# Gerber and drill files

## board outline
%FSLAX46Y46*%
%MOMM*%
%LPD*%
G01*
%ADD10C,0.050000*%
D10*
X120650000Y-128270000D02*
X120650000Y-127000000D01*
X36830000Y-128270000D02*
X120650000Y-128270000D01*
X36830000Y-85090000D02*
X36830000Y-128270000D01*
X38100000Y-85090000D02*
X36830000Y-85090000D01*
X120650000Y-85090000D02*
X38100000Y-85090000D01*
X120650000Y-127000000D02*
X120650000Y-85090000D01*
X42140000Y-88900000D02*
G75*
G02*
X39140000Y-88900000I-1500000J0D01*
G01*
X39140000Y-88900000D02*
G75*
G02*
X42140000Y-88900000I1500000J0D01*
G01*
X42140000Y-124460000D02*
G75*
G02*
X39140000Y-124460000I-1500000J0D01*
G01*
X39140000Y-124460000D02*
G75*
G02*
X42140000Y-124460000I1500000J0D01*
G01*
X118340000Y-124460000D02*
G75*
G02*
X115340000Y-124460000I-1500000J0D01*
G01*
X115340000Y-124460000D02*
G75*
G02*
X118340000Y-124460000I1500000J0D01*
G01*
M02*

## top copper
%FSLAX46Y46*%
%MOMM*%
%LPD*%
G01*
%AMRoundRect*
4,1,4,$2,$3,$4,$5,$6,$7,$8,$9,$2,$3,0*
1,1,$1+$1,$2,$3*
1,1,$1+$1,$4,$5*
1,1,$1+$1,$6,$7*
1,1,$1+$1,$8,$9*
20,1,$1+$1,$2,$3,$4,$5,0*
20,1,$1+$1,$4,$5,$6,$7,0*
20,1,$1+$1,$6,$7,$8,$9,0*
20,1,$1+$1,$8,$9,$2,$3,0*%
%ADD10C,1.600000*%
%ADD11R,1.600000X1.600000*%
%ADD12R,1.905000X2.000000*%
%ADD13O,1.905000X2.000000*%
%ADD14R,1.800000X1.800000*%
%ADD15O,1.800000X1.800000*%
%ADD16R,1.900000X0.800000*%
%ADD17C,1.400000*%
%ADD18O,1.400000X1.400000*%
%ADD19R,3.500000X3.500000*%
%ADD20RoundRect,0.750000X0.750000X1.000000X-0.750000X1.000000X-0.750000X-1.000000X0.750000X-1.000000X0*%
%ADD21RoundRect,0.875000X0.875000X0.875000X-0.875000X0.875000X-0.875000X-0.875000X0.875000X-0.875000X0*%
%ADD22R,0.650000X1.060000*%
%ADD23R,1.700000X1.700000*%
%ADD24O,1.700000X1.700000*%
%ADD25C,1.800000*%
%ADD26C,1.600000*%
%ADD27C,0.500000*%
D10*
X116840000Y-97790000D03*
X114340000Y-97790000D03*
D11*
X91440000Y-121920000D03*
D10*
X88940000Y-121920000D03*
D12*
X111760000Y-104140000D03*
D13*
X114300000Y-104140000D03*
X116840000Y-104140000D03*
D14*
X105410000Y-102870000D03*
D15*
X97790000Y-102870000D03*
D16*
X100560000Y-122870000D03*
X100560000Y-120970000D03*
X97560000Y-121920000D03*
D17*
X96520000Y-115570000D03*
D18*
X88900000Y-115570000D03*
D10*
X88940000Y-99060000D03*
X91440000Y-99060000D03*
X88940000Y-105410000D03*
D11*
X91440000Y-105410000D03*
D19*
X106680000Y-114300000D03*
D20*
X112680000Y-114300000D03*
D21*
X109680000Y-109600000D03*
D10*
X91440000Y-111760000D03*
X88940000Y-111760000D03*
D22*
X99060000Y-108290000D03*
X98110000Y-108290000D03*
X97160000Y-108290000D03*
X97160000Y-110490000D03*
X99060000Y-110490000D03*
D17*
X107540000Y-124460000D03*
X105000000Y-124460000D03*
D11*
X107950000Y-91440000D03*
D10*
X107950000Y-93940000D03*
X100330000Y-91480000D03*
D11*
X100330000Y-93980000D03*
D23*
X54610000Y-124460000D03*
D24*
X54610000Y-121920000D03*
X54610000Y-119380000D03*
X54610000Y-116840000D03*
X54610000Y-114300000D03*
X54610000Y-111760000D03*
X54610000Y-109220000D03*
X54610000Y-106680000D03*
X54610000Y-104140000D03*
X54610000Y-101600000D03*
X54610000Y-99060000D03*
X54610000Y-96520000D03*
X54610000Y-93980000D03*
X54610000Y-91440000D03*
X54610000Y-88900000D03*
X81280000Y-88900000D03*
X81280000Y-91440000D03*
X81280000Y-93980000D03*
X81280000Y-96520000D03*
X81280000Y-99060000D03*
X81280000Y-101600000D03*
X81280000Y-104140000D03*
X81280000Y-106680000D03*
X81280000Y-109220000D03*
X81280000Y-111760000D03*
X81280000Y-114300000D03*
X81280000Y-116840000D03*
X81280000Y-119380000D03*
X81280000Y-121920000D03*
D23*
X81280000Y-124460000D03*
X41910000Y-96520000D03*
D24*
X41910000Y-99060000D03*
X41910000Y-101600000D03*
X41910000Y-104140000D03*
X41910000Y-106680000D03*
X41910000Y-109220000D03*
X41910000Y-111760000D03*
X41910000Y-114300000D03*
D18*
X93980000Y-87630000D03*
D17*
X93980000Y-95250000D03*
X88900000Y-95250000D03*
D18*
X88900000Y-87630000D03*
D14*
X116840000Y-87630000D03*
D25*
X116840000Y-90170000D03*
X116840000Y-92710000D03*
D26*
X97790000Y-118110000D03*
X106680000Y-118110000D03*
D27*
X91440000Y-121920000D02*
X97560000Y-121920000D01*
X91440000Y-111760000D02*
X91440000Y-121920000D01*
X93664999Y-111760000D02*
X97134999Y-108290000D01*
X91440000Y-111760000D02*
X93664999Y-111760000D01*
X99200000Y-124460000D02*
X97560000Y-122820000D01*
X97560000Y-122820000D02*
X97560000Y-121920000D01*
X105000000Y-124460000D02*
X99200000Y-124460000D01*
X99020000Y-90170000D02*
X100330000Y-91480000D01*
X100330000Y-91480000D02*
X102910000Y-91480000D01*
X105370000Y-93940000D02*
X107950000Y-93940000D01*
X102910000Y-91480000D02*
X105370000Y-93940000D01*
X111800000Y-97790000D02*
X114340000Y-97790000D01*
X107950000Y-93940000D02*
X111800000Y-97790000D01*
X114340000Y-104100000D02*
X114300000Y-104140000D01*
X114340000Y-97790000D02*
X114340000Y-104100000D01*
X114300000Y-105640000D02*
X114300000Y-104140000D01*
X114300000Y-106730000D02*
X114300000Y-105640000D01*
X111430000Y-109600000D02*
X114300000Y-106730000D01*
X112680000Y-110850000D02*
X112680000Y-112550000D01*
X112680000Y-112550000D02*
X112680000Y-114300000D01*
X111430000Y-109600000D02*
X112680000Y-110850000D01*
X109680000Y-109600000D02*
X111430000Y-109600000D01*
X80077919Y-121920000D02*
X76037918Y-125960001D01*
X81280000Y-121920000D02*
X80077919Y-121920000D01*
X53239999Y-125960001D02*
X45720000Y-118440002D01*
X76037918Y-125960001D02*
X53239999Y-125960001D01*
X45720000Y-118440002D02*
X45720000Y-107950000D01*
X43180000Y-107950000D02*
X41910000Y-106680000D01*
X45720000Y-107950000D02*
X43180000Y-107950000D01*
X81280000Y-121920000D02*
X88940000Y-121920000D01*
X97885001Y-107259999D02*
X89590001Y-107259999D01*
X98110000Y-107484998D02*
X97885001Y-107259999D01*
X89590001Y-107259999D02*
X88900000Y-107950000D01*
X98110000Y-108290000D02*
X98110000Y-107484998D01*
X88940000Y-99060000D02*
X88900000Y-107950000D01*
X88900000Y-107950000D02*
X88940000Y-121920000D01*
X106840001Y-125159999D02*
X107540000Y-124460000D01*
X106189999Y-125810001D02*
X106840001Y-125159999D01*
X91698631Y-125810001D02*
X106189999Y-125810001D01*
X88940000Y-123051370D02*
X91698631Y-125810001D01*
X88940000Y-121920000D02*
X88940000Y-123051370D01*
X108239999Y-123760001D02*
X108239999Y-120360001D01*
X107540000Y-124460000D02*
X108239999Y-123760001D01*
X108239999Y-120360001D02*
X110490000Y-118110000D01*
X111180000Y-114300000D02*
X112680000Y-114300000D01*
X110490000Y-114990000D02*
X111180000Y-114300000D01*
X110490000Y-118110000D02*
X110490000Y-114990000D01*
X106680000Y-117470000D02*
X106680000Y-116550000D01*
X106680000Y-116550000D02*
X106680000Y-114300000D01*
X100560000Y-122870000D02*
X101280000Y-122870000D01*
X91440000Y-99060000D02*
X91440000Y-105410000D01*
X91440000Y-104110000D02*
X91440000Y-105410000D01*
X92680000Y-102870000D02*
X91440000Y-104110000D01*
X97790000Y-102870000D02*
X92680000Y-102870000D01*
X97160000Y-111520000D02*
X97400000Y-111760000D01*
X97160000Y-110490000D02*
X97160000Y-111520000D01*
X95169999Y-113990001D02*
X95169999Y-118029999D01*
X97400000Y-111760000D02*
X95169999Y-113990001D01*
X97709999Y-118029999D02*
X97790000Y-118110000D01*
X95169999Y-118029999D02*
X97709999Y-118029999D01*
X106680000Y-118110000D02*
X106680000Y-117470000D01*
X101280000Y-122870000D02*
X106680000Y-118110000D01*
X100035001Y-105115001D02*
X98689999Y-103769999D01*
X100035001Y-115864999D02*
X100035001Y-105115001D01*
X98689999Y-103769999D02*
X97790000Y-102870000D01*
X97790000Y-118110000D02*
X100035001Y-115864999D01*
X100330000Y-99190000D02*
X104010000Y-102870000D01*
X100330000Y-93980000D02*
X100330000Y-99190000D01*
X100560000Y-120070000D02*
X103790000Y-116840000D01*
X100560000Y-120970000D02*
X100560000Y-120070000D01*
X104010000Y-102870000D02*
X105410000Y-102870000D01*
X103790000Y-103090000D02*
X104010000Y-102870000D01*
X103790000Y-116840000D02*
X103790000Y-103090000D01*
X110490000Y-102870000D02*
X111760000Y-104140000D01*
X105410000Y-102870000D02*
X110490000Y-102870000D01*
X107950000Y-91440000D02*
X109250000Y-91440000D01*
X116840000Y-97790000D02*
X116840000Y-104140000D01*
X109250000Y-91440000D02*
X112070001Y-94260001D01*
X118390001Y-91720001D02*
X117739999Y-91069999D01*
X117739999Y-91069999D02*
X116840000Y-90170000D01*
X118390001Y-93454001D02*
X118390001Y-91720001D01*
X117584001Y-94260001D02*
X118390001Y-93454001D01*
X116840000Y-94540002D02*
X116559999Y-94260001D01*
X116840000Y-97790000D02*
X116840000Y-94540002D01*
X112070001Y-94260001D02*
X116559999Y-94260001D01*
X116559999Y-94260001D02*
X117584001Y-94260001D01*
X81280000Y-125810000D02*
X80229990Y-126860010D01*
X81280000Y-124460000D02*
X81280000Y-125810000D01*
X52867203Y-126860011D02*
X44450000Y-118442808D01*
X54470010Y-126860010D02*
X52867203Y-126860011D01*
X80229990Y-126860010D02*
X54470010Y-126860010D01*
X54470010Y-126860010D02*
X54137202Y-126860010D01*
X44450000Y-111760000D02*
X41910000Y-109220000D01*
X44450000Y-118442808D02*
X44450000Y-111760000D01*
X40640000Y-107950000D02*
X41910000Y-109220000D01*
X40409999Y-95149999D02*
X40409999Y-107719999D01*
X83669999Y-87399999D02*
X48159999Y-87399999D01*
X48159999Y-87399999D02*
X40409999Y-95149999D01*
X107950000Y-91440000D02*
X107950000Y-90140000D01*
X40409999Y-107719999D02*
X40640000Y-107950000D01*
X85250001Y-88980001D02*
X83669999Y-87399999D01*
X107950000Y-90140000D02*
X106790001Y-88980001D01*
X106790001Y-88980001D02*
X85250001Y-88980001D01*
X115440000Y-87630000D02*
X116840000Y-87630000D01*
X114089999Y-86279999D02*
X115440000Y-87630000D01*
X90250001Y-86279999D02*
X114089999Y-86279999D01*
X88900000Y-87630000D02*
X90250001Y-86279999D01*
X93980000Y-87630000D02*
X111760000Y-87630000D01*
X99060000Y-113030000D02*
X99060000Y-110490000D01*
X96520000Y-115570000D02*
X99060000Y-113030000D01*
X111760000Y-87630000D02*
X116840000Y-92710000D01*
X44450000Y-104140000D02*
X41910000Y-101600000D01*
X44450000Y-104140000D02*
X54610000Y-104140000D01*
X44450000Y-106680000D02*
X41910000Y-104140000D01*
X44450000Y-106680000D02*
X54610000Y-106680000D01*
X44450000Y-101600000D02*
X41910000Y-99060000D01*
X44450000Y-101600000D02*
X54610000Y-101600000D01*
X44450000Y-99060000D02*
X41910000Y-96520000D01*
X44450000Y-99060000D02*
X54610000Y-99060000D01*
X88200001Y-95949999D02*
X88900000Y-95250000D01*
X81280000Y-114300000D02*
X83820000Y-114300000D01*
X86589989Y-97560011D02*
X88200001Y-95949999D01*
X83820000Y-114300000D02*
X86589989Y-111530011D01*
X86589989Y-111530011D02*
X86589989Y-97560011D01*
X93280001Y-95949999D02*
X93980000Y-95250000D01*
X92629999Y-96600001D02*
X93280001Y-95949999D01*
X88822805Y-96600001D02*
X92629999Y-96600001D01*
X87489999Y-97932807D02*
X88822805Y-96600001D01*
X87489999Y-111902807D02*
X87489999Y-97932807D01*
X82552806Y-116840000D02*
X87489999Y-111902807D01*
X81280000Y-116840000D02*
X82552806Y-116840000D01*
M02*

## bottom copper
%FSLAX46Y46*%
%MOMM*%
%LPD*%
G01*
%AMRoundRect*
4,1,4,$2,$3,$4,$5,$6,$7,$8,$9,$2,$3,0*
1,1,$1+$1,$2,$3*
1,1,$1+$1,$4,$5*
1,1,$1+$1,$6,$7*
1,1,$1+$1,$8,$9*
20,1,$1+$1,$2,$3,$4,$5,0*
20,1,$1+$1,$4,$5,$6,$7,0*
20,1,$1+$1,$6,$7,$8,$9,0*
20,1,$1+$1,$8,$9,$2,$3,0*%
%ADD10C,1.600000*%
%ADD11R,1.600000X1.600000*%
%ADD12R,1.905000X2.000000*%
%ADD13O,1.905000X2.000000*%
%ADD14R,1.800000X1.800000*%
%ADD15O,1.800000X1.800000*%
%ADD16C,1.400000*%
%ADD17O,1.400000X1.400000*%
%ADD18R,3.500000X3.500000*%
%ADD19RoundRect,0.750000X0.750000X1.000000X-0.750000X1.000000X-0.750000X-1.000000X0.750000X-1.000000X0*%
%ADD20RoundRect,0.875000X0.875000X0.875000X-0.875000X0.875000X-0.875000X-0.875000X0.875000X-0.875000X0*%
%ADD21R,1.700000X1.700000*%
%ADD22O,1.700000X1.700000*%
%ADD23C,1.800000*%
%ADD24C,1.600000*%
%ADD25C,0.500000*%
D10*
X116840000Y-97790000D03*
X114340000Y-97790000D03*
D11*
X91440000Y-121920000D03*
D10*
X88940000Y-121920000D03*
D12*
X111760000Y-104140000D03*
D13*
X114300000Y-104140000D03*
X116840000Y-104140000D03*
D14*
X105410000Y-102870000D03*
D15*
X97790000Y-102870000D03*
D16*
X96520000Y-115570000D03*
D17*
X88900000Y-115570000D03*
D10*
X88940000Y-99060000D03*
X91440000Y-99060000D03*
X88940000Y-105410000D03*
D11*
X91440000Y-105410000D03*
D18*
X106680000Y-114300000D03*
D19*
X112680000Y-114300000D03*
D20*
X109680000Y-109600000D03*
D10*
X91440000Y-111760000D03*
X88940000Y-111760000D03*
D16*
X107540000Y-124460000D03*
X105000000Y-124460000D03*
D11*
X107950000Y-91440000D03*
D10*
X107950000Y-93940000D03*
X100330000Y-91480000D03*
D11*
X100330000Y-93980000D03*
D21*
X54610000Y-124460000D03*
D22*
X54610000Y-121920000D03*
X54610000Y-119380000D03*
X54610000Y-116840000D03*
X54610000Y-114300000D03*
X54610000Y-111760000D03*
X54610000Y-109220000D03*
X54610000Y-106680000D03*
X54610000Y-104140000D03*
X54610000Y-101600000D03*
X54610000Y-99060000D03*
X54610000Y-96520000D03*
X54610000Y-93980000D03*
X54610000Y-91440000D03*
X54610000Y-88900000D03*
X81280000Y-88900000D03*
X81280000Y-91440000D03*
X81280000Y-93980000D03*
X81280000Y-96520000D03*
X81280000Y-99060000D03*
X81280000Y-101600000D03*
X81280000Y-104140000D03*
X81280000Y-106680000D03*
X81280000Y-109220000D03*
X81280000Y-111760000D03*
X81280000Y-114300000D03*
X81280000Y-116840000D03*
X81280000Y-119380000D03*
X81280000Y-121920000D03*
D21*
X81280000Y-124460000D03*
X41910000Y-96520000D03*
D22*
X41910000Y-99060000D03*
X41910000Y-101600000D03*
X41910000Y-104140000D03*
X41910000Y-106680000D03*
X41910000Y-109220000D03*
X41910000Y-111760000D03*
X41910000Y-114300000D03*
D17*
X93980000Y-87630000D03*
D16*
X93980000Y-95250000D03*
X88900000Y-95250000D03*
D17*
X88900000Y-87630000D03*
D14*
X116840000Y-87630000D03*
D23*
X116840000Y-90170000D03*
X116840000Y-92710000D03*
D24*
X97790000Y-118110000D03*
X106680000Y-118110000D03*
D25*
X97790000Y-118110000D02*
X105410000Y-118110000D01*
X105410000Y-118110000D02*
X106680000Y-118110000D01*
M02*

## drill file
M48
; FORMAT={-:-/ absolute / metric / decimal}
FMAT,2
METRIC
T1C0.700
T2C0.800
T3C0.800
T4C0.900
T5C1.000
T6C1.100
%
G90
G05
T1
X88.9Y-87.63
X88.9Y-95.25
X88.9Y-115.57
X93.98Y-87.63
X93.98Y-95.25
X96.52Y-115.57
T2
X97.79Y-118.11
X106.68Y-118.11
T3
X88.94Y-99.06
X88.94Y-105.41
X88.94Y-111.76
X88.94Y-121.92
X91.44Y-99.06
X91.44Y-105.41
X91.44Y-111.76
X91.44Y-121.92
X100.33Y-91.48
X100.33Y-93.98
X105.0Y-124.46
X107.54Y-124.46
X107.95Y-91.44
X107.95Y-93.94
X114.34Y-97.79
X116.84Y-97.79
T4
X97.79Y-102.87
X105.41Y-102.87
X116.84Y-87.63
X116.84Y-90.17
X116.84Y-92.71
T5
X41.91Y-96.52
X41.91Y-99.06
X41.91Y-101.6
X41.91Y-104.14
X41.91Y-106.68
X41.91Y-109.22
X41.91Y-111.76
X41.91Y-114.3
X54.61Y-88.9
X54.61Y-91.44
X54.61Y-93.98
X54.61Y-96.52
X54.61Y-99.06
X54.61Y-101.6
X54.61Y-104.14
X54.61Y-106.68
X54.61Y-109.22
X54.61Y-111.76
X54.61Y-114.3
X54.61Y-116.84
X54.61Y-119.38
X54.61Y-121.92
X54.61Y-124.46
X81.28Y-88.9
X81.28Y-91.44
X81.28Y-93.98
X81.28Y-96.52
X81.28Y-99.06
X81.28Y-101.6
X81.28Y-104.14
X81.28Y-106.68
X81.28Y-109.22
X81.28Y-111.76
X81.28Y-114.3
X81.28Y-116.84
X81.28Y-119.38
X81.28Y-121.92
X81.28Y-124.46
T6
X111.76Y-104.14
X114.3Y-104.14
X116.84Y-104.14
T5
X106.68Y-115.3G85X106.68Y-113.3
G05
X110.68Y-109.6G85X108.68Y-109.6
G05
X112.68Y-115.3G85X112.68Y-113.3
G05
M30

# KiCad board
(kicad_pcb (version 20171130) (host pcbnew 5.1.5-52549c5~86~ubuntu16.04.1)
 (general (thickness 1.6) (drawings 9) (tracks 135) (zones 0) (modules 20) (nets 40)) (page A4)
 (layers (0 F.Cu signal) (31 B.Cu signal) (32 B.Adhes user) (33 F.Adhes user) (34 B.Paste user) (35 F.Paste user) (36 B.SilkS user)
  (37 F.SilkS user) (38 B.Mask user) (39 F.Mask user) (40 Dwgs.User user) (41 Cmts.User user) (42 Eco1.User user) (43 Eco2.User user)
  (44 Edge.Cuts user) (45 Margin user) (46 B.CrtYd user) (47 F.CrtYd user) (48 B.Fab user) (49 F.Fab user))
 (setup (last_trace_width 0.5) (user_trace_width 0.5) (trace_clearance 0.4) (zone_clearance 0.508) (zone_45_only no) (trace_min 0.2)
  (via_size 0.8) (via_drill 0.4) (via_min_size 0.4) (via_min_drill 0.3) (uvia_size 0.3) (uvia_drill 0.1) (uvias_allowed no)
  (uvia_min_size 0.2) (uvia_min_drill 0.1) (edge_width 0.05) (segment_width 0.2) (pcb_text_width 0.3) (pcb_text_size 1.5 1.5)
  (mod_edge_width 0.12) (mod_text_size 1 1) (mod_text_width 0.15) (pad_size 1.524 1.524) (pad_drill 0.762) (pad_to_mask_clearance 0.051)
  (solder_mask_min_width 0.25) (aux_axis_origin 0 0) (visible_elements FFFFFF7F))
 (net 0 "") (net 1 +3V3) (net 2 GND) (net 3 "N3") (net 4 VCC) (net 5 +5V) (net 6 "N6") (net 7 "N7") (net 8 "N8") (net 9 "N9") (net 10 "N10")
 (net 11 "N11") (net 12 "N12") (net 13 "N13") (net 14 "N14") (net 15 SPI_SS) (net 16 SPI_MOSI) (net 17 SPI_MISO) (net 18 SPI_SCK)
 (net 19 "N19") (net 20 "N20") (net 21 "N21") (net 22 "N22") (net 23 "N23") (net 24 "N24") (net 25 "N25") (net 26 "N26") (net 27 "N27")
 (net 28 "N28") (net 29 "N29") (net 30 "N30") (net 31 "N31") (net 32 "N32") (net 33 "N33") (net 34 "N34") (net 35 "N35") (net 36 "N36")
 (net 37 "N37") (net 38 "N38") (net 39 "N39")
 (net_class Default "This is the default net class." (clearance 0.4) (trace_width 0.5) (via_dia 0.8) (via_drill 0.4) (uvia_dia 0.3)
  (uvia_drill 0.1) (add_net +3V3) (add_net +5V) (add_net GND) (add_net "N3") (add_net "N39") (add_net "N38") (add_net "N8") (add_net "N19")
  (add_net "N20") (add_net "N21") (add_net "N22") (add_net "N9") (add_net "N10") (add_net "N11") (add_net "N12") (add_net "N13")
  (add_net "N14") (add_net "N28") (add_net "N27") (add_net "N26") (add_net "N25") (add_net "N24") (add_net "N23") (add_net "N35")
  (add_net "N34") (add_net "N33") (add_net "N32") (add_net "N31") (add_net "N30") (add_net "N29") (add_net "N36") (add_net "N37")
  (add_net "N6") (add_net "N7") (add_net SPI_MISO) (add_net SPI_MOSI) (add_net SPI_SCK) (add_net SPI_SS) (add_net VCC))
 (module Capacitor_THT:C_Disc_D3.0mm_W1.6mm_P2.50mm (layer F.Cu) (at 116.84 97.79 180)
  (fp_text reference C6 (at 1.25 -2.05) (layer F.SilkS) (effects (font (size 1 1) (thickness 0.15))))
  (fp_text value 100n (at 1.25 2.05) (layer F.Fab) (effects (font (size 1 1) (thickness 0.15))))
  (pad 1 thru_hole circle (at 0 0 180) (size 1.6 1.6) (drill 0.8) (layers *.Cu *.Mask) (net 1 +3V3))
  (pad 2 thru_hole circle (at 2.5 0 180) (size 1.6 1.6) (drill 0.8) (layers *.Cu *.Mask) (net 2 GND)))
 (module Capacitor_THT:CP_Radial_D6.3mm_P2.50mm (layer F.Cu) (at 91.44 121.92 180)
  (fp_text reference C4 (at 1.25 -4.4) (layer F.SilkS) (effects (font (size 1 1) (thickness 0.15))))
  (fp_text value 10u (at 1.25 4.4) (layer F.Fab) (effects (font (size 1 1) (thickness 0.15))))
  (pad 1 thru_hole rect (at 0 0 180) (size 1.6 1.6) (drill 0.8) (layers *.Cu *.Mask) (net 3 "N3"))
  (pad 2 thru_hole circle (at 2.5 0 180) (size 1.6 1.6) (drill 0.8) (layers *.Cu *.Mask) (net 2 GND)))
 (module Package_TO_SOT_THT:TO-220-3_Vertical (layer F.Cu) (at 111.76 104.14)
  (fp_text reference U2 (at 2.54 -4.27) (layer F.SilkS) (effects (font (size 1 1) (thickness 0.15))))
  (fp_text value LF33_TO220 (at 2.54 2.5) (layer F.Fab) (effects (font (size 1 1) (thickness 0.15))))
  (pad 1 thru_hole rect (at 0 0) (size 1.905 2) (drill 1.1) (layers *.Cu *.Mask) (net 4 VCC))
  (pad 2 thru_hole oval (at 2.54 0) (size 1.905 2) (drill 1.1) (layers *.Cu *.Mask) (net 2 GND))
  (pad 3 thru_hole oval (at 5.08 0) (size 1.905 2) (drill 1.1) (layers *.Cu *.Mask) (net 1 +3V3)))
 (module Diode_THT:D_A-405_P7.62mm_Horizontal (layer F.Cu) (at 105.41 102.87 180)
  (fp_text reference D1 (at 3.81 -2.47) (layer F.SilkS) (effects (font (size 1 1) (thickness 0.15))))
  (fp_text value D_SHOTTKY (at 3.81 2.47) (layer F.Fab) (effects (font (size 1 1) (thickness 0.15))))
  (pad 1 thru_hole rect (at 0 0 180) (size 1.8 1.8) (drill 0.9) (layers *.Cu *.Mask) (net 4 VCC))
  (pad 2 thru_hole oval (at 7.62 0 180) (size 1.8 1.8) (drill 0.9) (layers *.Cu *.Mask) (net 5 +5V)))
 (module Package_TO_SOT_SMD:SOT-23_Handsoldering (layer F.Cu) (at 99.06 121.92 180)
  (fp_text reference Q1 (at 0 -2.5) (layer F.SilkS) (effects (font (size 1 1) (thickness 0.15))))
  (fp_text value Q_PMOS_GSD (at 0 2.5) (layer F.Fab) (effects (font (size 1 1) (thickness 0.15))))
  (pad 1 smd rect (at -1.5 -0.95 180) (size 1.9 0.8) (layers F.Cu F.Paste F.Mask) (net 5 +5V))
  (pad 2 smd rect (at -1.5 0.95 180) (size 1.9 0.8) (layers F.Cu F.Paste F.Mask) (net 4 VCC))
  (pad 3 smd rect (at 1.5 0 180) (size 1.9 0.8) (layers F.Cu F.Paste F.Mask) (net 3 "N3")))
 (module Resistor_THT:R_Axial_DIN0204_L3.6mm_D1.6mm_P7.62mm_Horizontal (layer F.Cu) (at 96.52 115.57 180)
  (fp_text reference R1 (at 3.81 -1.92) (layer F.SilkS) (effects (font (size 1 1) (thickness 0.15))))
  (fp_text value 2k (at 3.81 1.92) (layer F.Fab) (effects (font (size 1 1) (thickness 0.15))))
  (pad 1 thru_hole circle (at 0 0 180) (size 1.4 1.4) (drill 0.7) (layers *.Cu *.Mask) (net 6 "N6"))
  (pad 2 thru_hole oval (at 7.62 0 180) (size 1.4 1.4) (drill 0.7) (layers *.Cu *.Mask) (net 2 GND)))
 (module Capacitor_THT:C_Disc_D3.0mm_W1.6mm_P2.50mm (layer F.Cu) (at 91.44 99.06 180)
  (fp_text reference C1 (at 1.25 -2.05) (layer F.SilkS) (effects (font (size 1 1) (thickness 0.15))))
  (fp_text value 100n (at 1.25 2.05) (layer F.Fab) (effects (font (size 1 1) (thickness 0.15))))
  (pad 2 thru_hole circle (at 2.5 0 180) (size 1.6 1.6) (drill 0.8) (layers *.Cu *.Mask) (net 2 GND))
  (pad 1 thru_hole circle (at 0 0 180) (size 1.6 1.6) (drill 0.8) (layers *.Cu *.Mask) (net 5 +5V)))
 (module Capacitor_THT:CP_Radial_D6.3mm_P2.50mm (layer F.Cu) (at 91.44 105.41 180)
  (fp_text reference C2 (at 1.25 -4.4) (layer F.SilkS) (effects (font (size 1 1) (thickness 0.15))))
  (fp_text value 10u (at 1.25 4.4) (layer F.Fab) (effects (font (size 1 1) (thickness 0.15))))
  (pad 2 thru_hole circle (at 2.5 0 180) (size 1.6 1.6) (drill 0.8) (layers *.Cu *.Mask) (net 2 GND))
  (pad 1 thru_hole rect (at 0 0 180) (size 1.6 1.6) (drill 0.8) (layers *.Cu *.Mask) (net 5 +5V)))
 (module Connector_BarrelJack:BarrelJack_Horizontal (layer F.Cu) (at 106.68 114.3 180)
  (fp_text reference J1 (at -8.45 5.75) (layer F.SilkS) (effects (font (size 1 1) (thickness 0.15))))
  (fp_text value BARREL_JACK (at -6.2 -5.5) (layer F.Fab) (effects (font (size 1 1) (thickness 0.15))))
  (pad 1 thru_hole rect (at 0 0 180) (size 3.5 3.5) (drill oval 1 3) (layers *.Cu *.Mask) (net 5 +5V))
  (pad 2 thru_hole roundrect (at -6 0 180) (size 3 3.5) (drill oval 1 3) (layers *.Cu *.Mask) (roundrect_rratio 0.25) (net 2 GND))
  (pad 3 thru_hole roundrect (at -3 4.7 180) (size 3.5 3.5) (drill oval 3 1) (layers *.Cu *.Mask) (roundrect_rratio 0.25) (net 2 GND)))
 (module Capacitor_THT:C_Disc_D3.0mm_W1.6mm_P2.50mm (layer F.Cu) (at 91.44 111.76 180)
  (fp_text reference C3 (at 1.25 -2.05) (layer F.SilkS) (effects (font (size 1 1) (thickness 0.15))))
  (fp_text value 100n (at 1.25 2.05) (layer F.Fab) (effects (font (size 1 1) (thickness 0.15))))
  (pad 1 thru_hole circle (at 0 0 180) (size 1.6 1.6) (drill 0.8) (layers *.Cu *.Mask) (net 3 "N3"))
  (pad 2 thru_hole circle (at 2.5 0 180) (size 1.6 1.6) (drill 0.8) (layers *.Cu *.Mask) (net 2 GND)))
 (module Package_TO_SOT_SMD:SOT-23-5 (layer F.Cu) (at 98.11 109.39 270)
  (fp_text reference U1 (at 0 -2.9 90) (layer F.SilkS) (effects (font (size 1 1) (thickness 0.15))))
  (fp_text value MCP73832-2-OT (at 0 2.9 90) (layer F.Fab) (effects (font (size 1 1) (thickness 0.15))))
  (pad 1 smd rect (at -1.1 -0.95 270) (size 1.06 0.65) (layers F.Cu F.Paste F.Mask) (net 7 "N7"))
  (pad 2 smd rect (at -1.1 0 270) (size 1.06 0.65) (layers F.Cu F.Paste F.Mask) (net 2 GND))
  (pad 3 smd rect (at -1.1 0.95 270) (size 1.06 0.65) (layers F.Cu F.Paste F.Mask) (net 3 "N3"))
  (pad 4 smd rect (at 1.1 0.95 270) (size 1.06 0.65) (layers F.Cu F.Paste F.Mask) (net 5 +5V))
  (pad 5 smd rect (at 1.1 -0.95 270) (size 1.06 0.65) (layers F.Cu F.Paste F.Mask) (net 6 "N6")))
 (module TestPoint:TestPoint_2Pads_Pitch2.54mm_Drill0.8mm (layer F.Cu) (at 105 124.46)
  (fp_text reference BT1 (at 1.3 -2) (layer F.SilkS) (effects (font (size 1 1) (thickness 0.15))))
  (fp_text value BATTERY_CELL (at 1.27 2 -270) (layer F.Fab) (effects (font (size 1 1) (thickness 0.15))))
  (pad 2 thru_hole circle (at 2.54 0) (size 1.4 1.4) (drill 0.8) (layers *.Cu *.Mask) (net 2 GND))
  (pad 1 thru_hole circle (at 0 0) (size 1.4 1.4) (drill 0.8) (layers *.Cu *.Mask) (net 3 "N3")))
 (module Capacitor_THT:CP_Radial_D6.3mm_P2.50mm (layer F.Cu) (at 107.95 91.44 270)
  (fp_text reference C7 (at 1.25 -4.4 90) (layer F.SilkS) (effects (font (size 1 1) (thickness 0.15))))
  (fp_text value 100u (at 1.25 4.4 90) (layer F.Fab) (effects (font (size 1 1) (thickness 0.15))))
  (pad 1 thru_hole rect (at 0 0 270) (size 1.6 1.6) (drill 0.8) (layers *.Cu *.Mask) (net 1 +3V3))
  (pad 2 thru_hole circle (at 2.5 0 270) (size 1.6 1.6) (drill 0.8) (layers *.Cu *.Mask) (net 2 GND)))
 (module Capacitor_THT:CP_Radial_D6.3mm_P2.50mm (layer F.Cu) (at 100.33 93.98 90)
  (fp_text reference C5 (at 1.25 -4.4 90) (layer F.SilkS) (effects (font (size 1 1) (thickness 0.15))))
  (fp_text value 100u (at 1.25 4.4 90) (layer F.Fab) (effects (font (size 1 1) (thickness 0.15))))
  (pad 2 thru_hole circle (at 2.5 0 90) (size 1.6 1.6) (drill 0.8) (layers *.Cu *.Mask) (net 2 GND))
  (pad 1 thru_hole rect (at 0 0 90) (size 1.6 1.6) (drill 0.8) (layers *.Cu *.Mask) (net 4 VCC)))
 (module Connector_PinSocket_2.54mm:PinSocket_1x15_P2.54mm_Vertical (layer F.Cu) (at 54.61 124.46 180)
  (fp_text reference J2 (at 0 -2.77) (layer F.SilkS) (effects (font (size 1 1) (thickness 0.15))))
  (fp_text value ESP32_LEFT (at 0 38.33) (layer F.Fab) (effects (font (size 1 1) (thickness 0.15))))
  (pad 1 thru_hole rect (at 0 0 180) (size 1.7 1.7) (drill 1) (layers *.Cu *.Mask) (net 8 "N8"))
  (pad 2 thru_hole oval (at 0 2.54 180) (size 1.7 1.7) (drill 1) (layers *.Cu *.Mask) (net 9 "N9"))
  (pad 3 thru_hole oval (at 0 5.08 180) (size 1.7 1.7) (drill 1) (layers *.Cu *.Mask) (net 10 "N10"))
  (pad 4 thru_hole oval (at 0 7.62 180) (size 1.7 1.7) (drill 1) (layers *.Cu *.Mask) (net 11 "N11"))
  (pad 5 thru_hole oval (at 0 10.16 180) (size 1.7 1.7) (drill 1) (layers *.Cu *.Mask) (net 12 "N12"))
  (pad 6 thru_hole oval (at 0 12.7 180) (size 1.7 1.7) (drill 1) (layers *.Cu *.Mask) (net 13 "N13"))
  (pad 7 thru_hole oval (at 0 15.24 180) (size 1.7 1.7) (drill 1) (layers *.Cu *.Mask) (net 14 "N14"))
  (pad 8 thru_hole oval (at 0 17.78 180) (size 1.7 1.7) (drill 1) (layers *.Cu *.Mask) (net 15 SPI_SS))
  (pad 9 thru_hole oval (at 0 20.32 180) (size 1.7 1.7) (drill 1) (layers *.Cu *.Mask) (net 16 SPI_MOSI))
  (pad 10 thru_hole oval (at 0 22.86 180) (size 1.7 1.7) (drill 1) (layers *.Cu *.Mask) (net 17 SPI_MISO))
  (pad 11 thru_hole oval (at 0 25.4 180) (size 1.7 1.7) (drill 1) (layers *.Cu *.Mask) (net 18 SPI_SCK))
  (pad 12 thru_hole oval (at 0 27.94 180) (size 1.7 1.7) (drill 1) (layers *.Cu *.Mask) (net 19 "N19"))
  (pad 13 thru_hole oval (at 0 30.48 180) (size 1.7 1.7) (drill 1) (layers *.Cu *.Mask) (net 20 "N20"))
  (pad 14 thru_hole oval (at 0 33.02 180) (size 1.7 1.7) (drill 1) (layers *.Cu *.Mask) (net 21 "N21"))
  (pad 15 thru_hole oval (at 0 35.56 180) (size 1.7 1.7) (drill 1) (layers *.Cu *.Mask) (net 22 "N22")))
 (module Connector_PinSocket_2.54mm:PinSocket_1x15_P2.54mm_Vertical (layer F.Cu) (at 81.28 124.46 180)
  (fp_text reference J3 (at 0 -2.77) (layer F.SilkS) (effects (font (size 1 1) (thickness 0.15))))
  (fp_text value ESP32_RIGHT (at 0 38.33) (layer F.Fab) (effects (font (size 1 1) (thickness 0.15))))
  (pad 15 thru_hole oval (at 0 35.56 180) (size 1.7 1.7) (drill 1) (layers *.Cu *.Mask) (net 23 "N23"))
  (pad 14 thru_hole oval (at 0 33.02 180) (size 1.7 1.7) (drill 1) (layers *.Cu *.Mask) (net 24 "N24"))
  (pad 13 thru_hole oval (at 0 30.48 180) (size 1.7 1.7) (drill 1) (layers *.Cu *.Mask) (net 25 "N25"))
  (pad 12 thru_hole oval (at 0 27.94 180) (size 1.7 1.7) (drill 1) (layers *.Cu *.Mask) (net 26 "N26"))
  (pad 11 thru_hole oval (at 0 25.4 180) (size 1.7 1.7) (drill 1) (layers *.Cu *.Mask) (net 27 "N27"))
  (pad 10 thru_hole oval (at 0 22.86 180) (size 1.7 1.7) (drill 1) (layers *.Cu *.Mask) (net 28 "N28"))
  (pad 9 thru_hole oval (at 0 20.32 180) (size 1.7 1.7) (drill 1) (layers *.Cu *.Mask) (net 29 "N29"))
  (pad 8 thru_hole oval (at 0 17.78 180) (size 1.7 1.7) (drill 1) (layers *.Cu *.Mask) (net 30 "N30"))
  (pad 7 thru_hole oval (at 0 15.24 180) (size 1.7 1.7) (drill 1) (layers *.Cu *.Mask) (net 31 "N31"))
  (pad 6 thru_hole oval (at 0 12.7 180) (size 1.7 1.7) (drill 1) (layers *.Cu *.Mask) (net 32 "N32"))
  (pad 5 thru_hole oval (at 0 10.16 180) (size 1.7 1.7) (drill 1) (layers *.Cu *.Mask) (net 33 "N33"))
  (pad 4 thru_hole oval (at 0 7.62 180) (size 1.7 1.7) (drill 1) (layers *.Cu *.Mask) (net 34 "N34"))
  (pad 3 thru_hole oval (at 0 5.08 180) (size 1.7 1.7) (drill 1) (layers *.Cu *.Mask) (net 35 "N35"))
  (pad 2 thru_hole oval (at 0 2.54 180) (size 1.7 1.7) (drill 1) (layers *.Cu *.Mask) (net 2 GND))
  (pad 1 thru_hole rect (at 0 0 180) (size 1.7 1.7) (drill 1) (layers *.Cu *.Mask) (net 1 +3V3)))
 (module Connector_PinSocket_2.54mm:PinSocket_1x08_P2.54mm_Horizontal (layer F.Cu) (at 41.91 96.52)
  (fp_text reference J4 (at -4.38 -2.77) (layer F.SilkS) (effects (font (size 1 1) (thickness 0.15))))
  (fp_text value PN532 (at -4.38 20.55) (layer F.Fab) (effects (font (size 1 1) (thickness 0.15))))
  (pad 1 thru_hole rect (at 0 0) (size 1.7 1.7) (drill 1) (layers *.Cu *.Mask) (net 18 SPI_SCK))
  (pad 2 thru_hole oval (at 0 2.54) (size 1.7 1.7) (drill 1) (layers *.Cu *.Mask) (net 17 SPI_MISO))
  (pad 3 thru_hole oval (at 0 5.08) (size 1.7 1.7) (drill 1) (layers *.Cu *.Mask) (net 16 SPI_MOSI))
  (pad 4 thru_hole oval (at 0 7.62) (size 1.7 1.7) (drill 1) (layers *.Cu *.Mask) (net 15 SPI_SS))
  (pad 5 thru_hole oval (at 0 10.16) (size 1.7 1.7) (drill 1) (layers *.Cu *.Mask) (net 2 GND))
  (pad 6 thru_hole oval (at 0 12.7) (size 1.7 1.7) (drill 1) (layers *.Cu *.Mask) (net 1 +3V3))
  (pad 7 thru_hole oval (at 0 15.24) (size 1.7 1.7) (drill 1) (layers *.Cu *.Mask) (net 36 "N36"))
  (pad 8 thru_hole oval (at 0 17.78) (size 1.7 1.7) (drill 1) (layers *.Cu *.Mask) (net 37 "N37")))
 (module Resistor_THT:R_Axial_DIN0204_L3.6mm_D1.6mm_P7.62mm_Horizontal (layer F.Cu) (at 93.98 95.25 90)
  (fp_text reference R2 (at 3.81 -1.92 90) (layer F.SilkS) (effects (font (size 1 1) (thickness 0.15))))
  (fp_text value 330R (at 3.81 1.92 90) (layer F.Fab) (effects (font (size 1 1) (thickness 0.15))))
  (pad 2 thru_hole oval (at 7.62 0 90) (size 1.4 1.4) (drill 0.7) (layers *.Cu *.Mask) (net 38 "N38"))
  (pad 1 thru_hole circle (at 0 0 90) (size 1.4 1.4) (drill 0.7) (layers *.Cu *.Mask) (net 34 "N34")))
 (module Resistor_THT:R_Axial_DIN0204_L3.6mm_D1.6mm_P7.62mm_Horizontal (layer F.Cu) (at 88.9 95.25 90)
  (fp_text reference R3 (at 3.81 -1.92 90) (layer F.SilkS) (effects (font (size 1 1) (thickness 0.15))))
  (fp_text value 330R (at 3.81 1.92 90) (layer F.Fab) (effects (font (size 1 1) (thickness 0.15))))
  (pad 1 thru_hole circle (at 0 0 90) (size 1.4 1.4) (drill 0.7) (layers *.Cu *.Mask) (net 33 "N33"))
  (pad 2 thru_hole oval (at 7.62 0 90) (size 1.4 1.4) (drill 0.7) (layers *.Cu *.Mask) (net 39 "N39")))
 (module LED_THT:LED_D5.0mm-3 (layer F.Cu) (at 116.84 87.63 270)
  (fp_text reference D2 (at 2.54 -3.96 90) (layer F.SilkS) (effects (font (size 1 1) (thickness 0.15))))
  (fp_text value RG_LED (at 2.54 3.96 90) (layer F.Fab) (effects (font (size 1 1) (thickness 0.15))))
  (pad 1 thru_hole rect (at 0 0 270) (size 1.8 1.8) (drill 0.9) (layers *.Cu *.Mask) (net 39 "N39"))
  (pad 2 thru_hole circle (at 2.54 0 270) (size 1.8 1.8) (drill 0.9) (layers *.Cu *.Mask) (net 1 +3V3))
  (pad 3 thru_hole circle (at 5.08 0 270) (size 1.8 1.8) (drill 0.9) (layers *.Cu *.Mask) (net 38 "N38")))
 (gr_line (start 120.65 128.27) (end 120.65 127) (layer Edge.Cuts) (width 0.05))
 (gr_line (start 36.83 128.27) (end 120.65 128.27) (layer Edge.Cuts) (width 0.05))
 (gr_line (start 36.83 85.09) (end 36.83 128.27) (layer Edge.Cuts) (width 0.05))
 (gr_line (start 38.1 85.09) (end 36.83 85.09) (layer Edge.Cuts) (width 0.05))
 (gr_line (start 120.65 85.09) (end 38.1 85.09) (layer Edge.Cuts) (width 0.05))
 (gr_line (start 120.65 127) (end 120.65 85.09) (layer Edge.Cuts) (width 0.05))
 (gr_circle (center 40.64 88.9) (end 42.14 88.9) (layer Edge.Cuts) (width 0.05))
 (gr_circle (center 40.64 124.46) (end 42.14 124.46) (layer Edge.Cuts) (width 0.05))
 (gr_circle (center 116.84 124.46) (end 118.34 124.46) (layer Edge.Cuts) (width 0.05))
 (segment (start 91.44 121.92) (end 97.56 121.92) (width 0.5) (layer F.Cu) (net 3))
 (segment (start 91.44 111.76) (end 91.44 121.92) (width 0.5) (layer F.Cu) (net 3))
 (segment (start 93.664999 111.76) (end 97.134999 108.29) (width 0.5) (layer F.Cu) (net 3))
 (segment (start 91.44 111.76) (end 93.664999 111.76) (width 0.5) (layer F.Cu) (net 3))
 (segment (start 99.2 124.46) (end 97.56 122.82) (width 0.5) (layer F.Cu) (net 3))
 (segment (start 97.56 122.82) (end 97.56 121.92) (width 0.5) (layer F.Cu) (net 3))
 (segment (start 105 124.46) (end 99.2 124.46) (width 0.5) (layer F.Cu) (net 3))
 (segment (start 99.02 90.17) (end 100.33 91.48) (width 0.5) (layer F.Cu) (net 2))
 (segment (start 100.33 91.48) (end 102.91 91.48) (width 0.5) (layer F.Cu) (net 2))
 (segment (start 105.37 93.94) (end 107.95 93.94) (width 0.5) (layer F.Cu) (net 2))
 (segment (start 102.91 91.48) (end 105.37 93.94) (width 0.5) (layer F.Cu) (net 2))
 (segment (start 111.8 97.79) (end 114.34 97.79) (width 0.5) (layer F.Cu) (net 2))
 (segment (start 107.95 93.94) (end 111.8 97.79) (width 0.5) (layer F.Cu) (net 2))
 (segment (start 114.34 104.1) (end 114.3 104.14) (width 0.5) (layer F.Cu) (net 2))
 (segment (start 114.34 97.79) (end 114.34 104.1) (width 0.5) (layer F.Cu) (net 2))
 (segment (start 114.3 105.64) (end 114.3 104.14) (width 0.5) (layer F.Cu) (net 2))
 (segment (start 114.3 106.73) (end 114.3 105.64) (width 0.5) (layer F.Cu) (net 2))
 (segment (start 111.43 109.6) (end 114.3 106.73) (width 0.5) (layer F.Cu) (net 2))
 (segment (start 112.68 110.85) (end 112.68 112.55) (width 0.5) (layer F.Cu) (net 2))
 (segment (start 112.68 112.55) (end 112.68 114.3) (width 0.5) (layer F.Cu) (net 2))
 (segment (start 111.43 109.6) (end 112.68 110.85) (width 0.5) (layer F.Cu) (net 2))
 (segment (start 109.68 109.6) (end 111.43 109.6) (width 0.5) (layer F.Cu) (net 2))
 (segment (start 80.077919 121.92) (end 76.037918 125.960001) (width 0.5) (layer F.Cu) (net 2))
 (segment (start 81.28 121.92) (end 80.077919 121.92) (width 0.5) (layer F.Cu) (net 2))
 (segment (start 53.239999 125.960001) (end 45.72 118.440002) (width 0.5) (layer F.Cu) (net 2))
 (segment (start 76.037918 125.960001) (end 53.239999 125.960001) (width 0.5) (layer F.Cu) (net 2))
 (segment (start 45.72 118.440002) (end 45.72 107.95) (width 0.5) (layer F.Cu) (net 2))
 (segment (start 43.18 107.95) (end 41.91 106.68) (width 0.5) (layer F.Cu) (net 2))
 (segment (start 45.72 107.95) (end 43.18 107.95) (width 0.5) (layer F.Cu) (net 2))
 (segment (start 81.28 121.92) (end 88.94 121.92) (width 0.5) (layer F.Cu) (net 2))
 (segment (start 97.885001 107.259999) (end 89.590001 107.259999) (width 0.5) (layer F.Cu) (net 2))
 (segment (start 98.11 107.484998) (end 97.885001 107.259999) (width 0.5) (layer F.Cu) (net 2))
 (segment (start 89.590001 107.259999) (end 88.9 107.95) (width 0.5) (layer F.Cu) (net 2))
 (segment (start 98.11 108.29) (end 98.11 107.484998) (width 0.5) (layer F.Cu) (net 2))
 (segment (start 88.94 99.06) (end 88.9 107.95) (width 0.5) (layer F.Cu) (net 2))
 (segment (start 88.9 107.95) (end 88.94 121.92) (width 0.5) (layer F.Cu) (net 2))
 (segment (start 106.840001 125.159999) (end 107.54 124.46) (width 0.5) (layer F.Cu) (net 2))
 (segment (start 106.189999 125.810001) (end 106.840001 125.159999) (width 0.5) (layer F.Cu) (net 2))
 (segment (start 91.698631 125.810001) (end 106.189999 125.810001) (width 0.5) (layer F.Cu) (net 2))
 (segment (start 88.94 123.05137) (end 91.698631 125.810001) (width 0.5) (layer F.Cu) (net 2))
 (segment (start 88.94 121.92) (end 88.94 123.05137) (width 0.5) (layer F.Cu) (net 2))
 (segment (start 108.239999 123.760001) (end 108.239999 120.360001) (width 0.5) (layer F.Cu) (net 2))
 (segment (start 107.54 124.46) (end 108.239999 123.760001) (width 0.5) (layer F.Cu) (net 2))
 (segment (start 108.239999 120.360001) (end 110.49 118.11) (width 0.5) (layer F.Cu) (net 2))
 (segment (start 111.18 114.3) (end 112.68 114.3) (width 0.5) (layer F.Cu) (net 2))
 (segment (start 110.49 114.99) (end 111.18 114.3) (width 0.5) (layer F.Cu) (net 2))
 (segment (start 110.49 118.11) (end 110.49 114.99) (width 0.5) (layer F.Cu) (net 2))
 (segment (start 106.68 117.47) (end 106.68 116.55) (width 0.5) (layer F.Cu) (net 5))
 (segment (start 106.68 116.55) (end 106.68 114.3) (width 0.5) (layer F.Cu) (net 5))
 (segment (start 100.56 122.87) (end 101.28 122.87) (width 0.5) (layer F.Cu) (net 5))
 (segment (start 91.44 99.06) (end 91.44 105.41) (width 0.5) (layer F.Cu) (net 5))
 (segment (start 91.44 104.11) (end 91.44 105.41) (width 0.5) (layer F.Cu) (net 5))
 (segment (start 92.68 102.87) (end 91.44 104.11) (width 0.5) (layer F.Cu) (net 5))
 (segment (start 97.79 102.87) (end 92.68 102.87) (width 0.5) (layer F.Cu) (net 5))
 (segment (start 97.16 111.52) (end 97.4 111.76) (width 0.5) (layer F.Cu) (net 5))
 (segment (start 97.16 110.49) (end 97.16 111.52) (width 0.5) (layer F.Cu) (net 5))
 (segment (start 95.169999 113.990001) (end 95.169999 118.029999) (width 0.5) (layer F.Cu) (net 5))
 (segment (start 97.4 111.76) (end 95.169999 113.990001) (width 0.5) (layer F.Cu) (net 5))
 (via (at 97.79 118.11) (size 1.6) (drill 0.8) (layers F.Cu B.Cu) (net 5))
 (segment (start 97.709999 118.029999) (end 97.79 118.11) (width 0.5) (layer F.Cu) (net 5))
 (segment (start 95.169999 118.029999) (end 97.709999 118.029999) (width 0.5) (layer F.Cu) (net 5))
 (segment (start 97.79 118.11) (end 105.41 118.11) (width 0.5) (layer B.Cu) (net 5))
 (via (at 106.68 118.11) (size 1.6) (drill 0.8) (layers F.Cu B.Cu) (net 5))
 (segment (start 105.41 118.11) (end 106.68 118.11) (width 0.5) (layer B.Cu) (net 5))
 (segment (start 106.68 118.11) (end 106.68 117.47) (width 0.5) (layer F.Cu) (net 5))
 (segment (start 101.28 122.87) (end 106.68 118.11) (width 0.5) (layer F.Cu) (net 5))
 (segment (start 100.035001 105.115001) (end 98.689999 103.769999) (width 0.5) (layer F.Cu) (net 5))
 (segment (start 100.035001 115.864999) (end 100.035001 105.115001) (width 0.5) (layer F.Cu) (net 5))
 (segment (start 98.689999 103.769999) (end 97.79 102.87) (width 0.5) (layer F.Cu) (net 5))
 (segment (start 97.79 118.11) (end 100.035001 115.864999) (width 0.5) (layer F.Cu) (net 5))
 (segment (start 100.33 99.19) (end 104.01 102.87) (width 0.5) (layer F.Cu) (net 4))
 (segment (start 100.33 93.98) (end 100.33 99.19) (width 0.5) (layer F.Cu) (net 4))
 (segment (start 100.56 120.07) (end 103.79 116.84) (width 0.5) (layer F.Cu) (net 4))
 (segment (start 100.56 120.97) (end 100.56 120.07) (width 0.5) (layer F.Cu) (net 4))
 (segment (start 104.01 102.87) (end 105.41 102.87) (width 0.5) (layer F.Cu) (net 4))
 (segment (start 103.79 103.09) (end 104.01 102.87) (width 0.5) (layer F.Cu) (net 4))
 (segment (start 103.79 116.84) (end 103.79 103.09) (width 0.5) (layer F.Cu) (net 4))
 (segment (start 110.49 102.87) (end 111.76 104.14) (width 0.5) (layer F.Cu) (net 4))
 (segment (start 105.41 102.87) (end 110.49 102.87) (width 0.5) (layer F.Cu) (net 4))
 (segment (start 107.95 91.44) (end 109.25 91.44) (width 0.5) (layer F.Cu) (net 1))
 (segment (start 116.84 97.79) (end 116.84 104.14) (width 0.5) (layer F.Cu) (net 1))
 (segment (start 109.25 91.44) (end 112.070001 94.260001) (width 0.5) (layer F.Cu) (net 1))
 (segment (start 118.390001 91.720001) (end 117.739999 91.069999) (width 0.5) (layer F.Cu) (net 1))
 (segment (start 117.739999 91.069999) (end 116.84 90.17) (width 0.5) (layer F.Cu) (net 1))
 (segment (start 118.390001 93.454001) (end 118.390001 91.720001) (width 0.5) (layer F.Cu) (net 1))
 (segment (start 117.584001 94.260001) (end 118.390001 93.454001) (width 0.5) (layer F.Cu) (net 1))
 (segment (start 116.84 94.540002) (end 116.559999 94.260001) (width 0.5) (layer F.Cu) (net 1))
 (segment (start 116.84 97.79) (end 116.84 94.540002) (width 0.5) (layer F.Cu) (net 1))
 (segment (start 112.070001 94.260001) (end 116.559999 94.260001) (width 0.5) (layer F.Cu) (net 1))
 (segment (start 116.559999 94.260001) (end 117.584001 94.260001) (width 0.5) (layer F.Cu) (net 1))
 (segment (start 81.28 125.81) (end 80.22999 126.86001) (width 0.5) (layer F.Cu) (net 1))
 (segment (start 81.28 124.46) (end 81.28 125.81) (width 0.5) (layer F.Cu) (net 1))
 (segment (start 52.867203 126.860011) (end 44.45 118.442808) (width 0.5) (layer F.Cu) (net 1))
 (segment (start 54.47001 126.86001) (end 52.867203 126.860011) (width 0.5) (layer F.Cu) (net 1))
 (segment (start 80.22999 126.86001) (end 54.47001 126.86001) (width 0.5) (layer F.Cu) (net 1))
 (segment (start 54.47001 126.86001) (end 54.137202 126.86001) (width 0.5) (layer F.Cu) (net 1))
 (segment (start 44.45 111.76) (end 41.91 109.22) (width 0.5) (layer F.Cu) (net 1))
 (segment (start 44.45 118.442808) (end 44.45 111.76) (width 0.5) (layer F.Cu) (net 1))
 (segment (start 40.64 107.95) (end 41.91 109.22) (width 0.5) (layer F.Cu) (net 1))
 (segment (start 40.409999 95.149999) (end 40.409999 107.719999) (width 0.5) (layer F.Cu) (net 1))
 (segment (start 83.669999 87.399999) (end 48.159999 87.399999) (width 0.5) (layer F.Cu) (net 1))
 (segment (start 48.159999 87.399999) (end 40.409999 95.149999) (width 0.5) (layer F.Cu) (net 1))
 (segment (start 107.95 91.44) (end 107.95 90.14) (width 0.5) (layer F.Cu) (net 1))
 (segment (start 40.409999 107.719999) (end 40.64 107.95) (width 0.5) (layer F.Cu) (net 1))
 (segment (start 85.250001 88.980001) (end 83.669999 87.399999) (width 0.5) (layer F.Cu) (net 1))
 (segment (start 107.95 90.14) (end 106.790001 88.980001) (width 0.5) (layer F.Cu) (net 1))
 (segment (start 106.790001 88.980001) (end 85.250001 88.980001) (width 0.5) (layer F.Cu) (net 1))
 (segment (start 115.44 87.63) (end 116.84 87.63) (width 0.5) (layer F.Cu) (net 39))
 (segment (start 114.089999 86.279999) (end 115.44 87.63) (width 0.5) (layer F.Cu) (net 39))
 (segment (start 90.250001 86.279999) (end 114.089999 86.279999) (width 0.5) (layer F.Cu) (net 39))
 (segment (start 88.9 87.63) (end 90.250001 86.279999) (width 0.5) (layer F.Cu) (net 39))
 (segment (start 93.98 87.63) (end 111.76 87.63) (width 0.5) (layer F.Cu) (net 38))
 (segment (start 99.06 113.03) (end 99.06 110.49) (width 0.5) (layer F.Cu) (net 6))
 (segment (start 96.52 115.57) (end 99.06 113.03) (width 0.5) (layer F.Cu) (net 6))
 (segment (start 111.76 87.63) (end 116.84 92.71) (width 0.5) (layer F.Cu) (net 38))
 (segment (start 44.45 104.14) (end 41.91 101.6) (width 0.5) (layer F.Cu) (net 16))
 (segment (start 44.45 104.14) (end 54.61 104.14) (width 0.5) (layer F.Cu) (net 16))
 (segment (start 44.45 106.68) (end 41.91 104.14) (width 0.5) (layer F.Cu) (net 15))
 (segment (start 44.45 106.68) (end 54.61 106.68) (width 0.5) (layer F.Cu) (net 15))
 (segment (start 44.45 101.6) (end 41.91 99.06) (width 0.5) (layer F.Cu) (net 17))
 (segment (start 44.45 101.6) (end 54.61 101.6) (width 0.5) (layer F.Cu) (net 17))
 (segment (start 44.45 99.06) (end 41.91 96.52) (width 0.5) (layer F.Cu) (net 18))
 (segment (start 44.45 99.06) (end 54.61 99.06) (width 0.5) (layer F.Cu) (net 18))
 (segment (start 88.200001 95.949999) (end 88.9 95.25) (width 0.5) (layer F.Cu) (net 33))
 (segment (start 81.28 114.3) (end 83.82 114.3) (width 0.5) (layer F.Cu) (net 33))
 (segment (start 86.589989 97.560011) (end 88.200001 95.949999) (width 0.5) (layer F.Cu) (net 33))
 (segment (start 83.82 114.3) (end 86.589989 111.530011) (width 0.5) (layer F.Cu) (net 33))
 (segment (start 86.589989 111.530011) (end 86.589989 97.560011) (width 0.5) (layer F.Cu) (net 33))
 (segment (start 93.280001 95.949999) (end 93.98 95.25) (width 0.5) (layer F.Cu) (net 34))
 (segment (start 92.629999 96.600001) (end 93.280001 95.949999) (width 0.5) (layer F.Cu) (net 34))
 (segment (start 88.822805 96.600001) (end 92.629999 96.600001) (width 0.5) (layer F.Cu) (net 34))
 (segment (start 87.489999 97.932807) (end 88.822805 96.600001) (width 0.5) (layer F.Cu) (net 34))
 (segment (start 87.489999 111.902807) (end 87.489999 97.932807) (width 0.5) (layer F.Cu) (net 34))
 (segment (start 82.552806 116.84) (end 87.489999 111.902807) (width 0.5) (layer F.Cu) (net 34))
 (segment (start 81.28 116.84) (end 82.552806 116.84) (width 0.5) (layer F.Cu) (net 34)))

